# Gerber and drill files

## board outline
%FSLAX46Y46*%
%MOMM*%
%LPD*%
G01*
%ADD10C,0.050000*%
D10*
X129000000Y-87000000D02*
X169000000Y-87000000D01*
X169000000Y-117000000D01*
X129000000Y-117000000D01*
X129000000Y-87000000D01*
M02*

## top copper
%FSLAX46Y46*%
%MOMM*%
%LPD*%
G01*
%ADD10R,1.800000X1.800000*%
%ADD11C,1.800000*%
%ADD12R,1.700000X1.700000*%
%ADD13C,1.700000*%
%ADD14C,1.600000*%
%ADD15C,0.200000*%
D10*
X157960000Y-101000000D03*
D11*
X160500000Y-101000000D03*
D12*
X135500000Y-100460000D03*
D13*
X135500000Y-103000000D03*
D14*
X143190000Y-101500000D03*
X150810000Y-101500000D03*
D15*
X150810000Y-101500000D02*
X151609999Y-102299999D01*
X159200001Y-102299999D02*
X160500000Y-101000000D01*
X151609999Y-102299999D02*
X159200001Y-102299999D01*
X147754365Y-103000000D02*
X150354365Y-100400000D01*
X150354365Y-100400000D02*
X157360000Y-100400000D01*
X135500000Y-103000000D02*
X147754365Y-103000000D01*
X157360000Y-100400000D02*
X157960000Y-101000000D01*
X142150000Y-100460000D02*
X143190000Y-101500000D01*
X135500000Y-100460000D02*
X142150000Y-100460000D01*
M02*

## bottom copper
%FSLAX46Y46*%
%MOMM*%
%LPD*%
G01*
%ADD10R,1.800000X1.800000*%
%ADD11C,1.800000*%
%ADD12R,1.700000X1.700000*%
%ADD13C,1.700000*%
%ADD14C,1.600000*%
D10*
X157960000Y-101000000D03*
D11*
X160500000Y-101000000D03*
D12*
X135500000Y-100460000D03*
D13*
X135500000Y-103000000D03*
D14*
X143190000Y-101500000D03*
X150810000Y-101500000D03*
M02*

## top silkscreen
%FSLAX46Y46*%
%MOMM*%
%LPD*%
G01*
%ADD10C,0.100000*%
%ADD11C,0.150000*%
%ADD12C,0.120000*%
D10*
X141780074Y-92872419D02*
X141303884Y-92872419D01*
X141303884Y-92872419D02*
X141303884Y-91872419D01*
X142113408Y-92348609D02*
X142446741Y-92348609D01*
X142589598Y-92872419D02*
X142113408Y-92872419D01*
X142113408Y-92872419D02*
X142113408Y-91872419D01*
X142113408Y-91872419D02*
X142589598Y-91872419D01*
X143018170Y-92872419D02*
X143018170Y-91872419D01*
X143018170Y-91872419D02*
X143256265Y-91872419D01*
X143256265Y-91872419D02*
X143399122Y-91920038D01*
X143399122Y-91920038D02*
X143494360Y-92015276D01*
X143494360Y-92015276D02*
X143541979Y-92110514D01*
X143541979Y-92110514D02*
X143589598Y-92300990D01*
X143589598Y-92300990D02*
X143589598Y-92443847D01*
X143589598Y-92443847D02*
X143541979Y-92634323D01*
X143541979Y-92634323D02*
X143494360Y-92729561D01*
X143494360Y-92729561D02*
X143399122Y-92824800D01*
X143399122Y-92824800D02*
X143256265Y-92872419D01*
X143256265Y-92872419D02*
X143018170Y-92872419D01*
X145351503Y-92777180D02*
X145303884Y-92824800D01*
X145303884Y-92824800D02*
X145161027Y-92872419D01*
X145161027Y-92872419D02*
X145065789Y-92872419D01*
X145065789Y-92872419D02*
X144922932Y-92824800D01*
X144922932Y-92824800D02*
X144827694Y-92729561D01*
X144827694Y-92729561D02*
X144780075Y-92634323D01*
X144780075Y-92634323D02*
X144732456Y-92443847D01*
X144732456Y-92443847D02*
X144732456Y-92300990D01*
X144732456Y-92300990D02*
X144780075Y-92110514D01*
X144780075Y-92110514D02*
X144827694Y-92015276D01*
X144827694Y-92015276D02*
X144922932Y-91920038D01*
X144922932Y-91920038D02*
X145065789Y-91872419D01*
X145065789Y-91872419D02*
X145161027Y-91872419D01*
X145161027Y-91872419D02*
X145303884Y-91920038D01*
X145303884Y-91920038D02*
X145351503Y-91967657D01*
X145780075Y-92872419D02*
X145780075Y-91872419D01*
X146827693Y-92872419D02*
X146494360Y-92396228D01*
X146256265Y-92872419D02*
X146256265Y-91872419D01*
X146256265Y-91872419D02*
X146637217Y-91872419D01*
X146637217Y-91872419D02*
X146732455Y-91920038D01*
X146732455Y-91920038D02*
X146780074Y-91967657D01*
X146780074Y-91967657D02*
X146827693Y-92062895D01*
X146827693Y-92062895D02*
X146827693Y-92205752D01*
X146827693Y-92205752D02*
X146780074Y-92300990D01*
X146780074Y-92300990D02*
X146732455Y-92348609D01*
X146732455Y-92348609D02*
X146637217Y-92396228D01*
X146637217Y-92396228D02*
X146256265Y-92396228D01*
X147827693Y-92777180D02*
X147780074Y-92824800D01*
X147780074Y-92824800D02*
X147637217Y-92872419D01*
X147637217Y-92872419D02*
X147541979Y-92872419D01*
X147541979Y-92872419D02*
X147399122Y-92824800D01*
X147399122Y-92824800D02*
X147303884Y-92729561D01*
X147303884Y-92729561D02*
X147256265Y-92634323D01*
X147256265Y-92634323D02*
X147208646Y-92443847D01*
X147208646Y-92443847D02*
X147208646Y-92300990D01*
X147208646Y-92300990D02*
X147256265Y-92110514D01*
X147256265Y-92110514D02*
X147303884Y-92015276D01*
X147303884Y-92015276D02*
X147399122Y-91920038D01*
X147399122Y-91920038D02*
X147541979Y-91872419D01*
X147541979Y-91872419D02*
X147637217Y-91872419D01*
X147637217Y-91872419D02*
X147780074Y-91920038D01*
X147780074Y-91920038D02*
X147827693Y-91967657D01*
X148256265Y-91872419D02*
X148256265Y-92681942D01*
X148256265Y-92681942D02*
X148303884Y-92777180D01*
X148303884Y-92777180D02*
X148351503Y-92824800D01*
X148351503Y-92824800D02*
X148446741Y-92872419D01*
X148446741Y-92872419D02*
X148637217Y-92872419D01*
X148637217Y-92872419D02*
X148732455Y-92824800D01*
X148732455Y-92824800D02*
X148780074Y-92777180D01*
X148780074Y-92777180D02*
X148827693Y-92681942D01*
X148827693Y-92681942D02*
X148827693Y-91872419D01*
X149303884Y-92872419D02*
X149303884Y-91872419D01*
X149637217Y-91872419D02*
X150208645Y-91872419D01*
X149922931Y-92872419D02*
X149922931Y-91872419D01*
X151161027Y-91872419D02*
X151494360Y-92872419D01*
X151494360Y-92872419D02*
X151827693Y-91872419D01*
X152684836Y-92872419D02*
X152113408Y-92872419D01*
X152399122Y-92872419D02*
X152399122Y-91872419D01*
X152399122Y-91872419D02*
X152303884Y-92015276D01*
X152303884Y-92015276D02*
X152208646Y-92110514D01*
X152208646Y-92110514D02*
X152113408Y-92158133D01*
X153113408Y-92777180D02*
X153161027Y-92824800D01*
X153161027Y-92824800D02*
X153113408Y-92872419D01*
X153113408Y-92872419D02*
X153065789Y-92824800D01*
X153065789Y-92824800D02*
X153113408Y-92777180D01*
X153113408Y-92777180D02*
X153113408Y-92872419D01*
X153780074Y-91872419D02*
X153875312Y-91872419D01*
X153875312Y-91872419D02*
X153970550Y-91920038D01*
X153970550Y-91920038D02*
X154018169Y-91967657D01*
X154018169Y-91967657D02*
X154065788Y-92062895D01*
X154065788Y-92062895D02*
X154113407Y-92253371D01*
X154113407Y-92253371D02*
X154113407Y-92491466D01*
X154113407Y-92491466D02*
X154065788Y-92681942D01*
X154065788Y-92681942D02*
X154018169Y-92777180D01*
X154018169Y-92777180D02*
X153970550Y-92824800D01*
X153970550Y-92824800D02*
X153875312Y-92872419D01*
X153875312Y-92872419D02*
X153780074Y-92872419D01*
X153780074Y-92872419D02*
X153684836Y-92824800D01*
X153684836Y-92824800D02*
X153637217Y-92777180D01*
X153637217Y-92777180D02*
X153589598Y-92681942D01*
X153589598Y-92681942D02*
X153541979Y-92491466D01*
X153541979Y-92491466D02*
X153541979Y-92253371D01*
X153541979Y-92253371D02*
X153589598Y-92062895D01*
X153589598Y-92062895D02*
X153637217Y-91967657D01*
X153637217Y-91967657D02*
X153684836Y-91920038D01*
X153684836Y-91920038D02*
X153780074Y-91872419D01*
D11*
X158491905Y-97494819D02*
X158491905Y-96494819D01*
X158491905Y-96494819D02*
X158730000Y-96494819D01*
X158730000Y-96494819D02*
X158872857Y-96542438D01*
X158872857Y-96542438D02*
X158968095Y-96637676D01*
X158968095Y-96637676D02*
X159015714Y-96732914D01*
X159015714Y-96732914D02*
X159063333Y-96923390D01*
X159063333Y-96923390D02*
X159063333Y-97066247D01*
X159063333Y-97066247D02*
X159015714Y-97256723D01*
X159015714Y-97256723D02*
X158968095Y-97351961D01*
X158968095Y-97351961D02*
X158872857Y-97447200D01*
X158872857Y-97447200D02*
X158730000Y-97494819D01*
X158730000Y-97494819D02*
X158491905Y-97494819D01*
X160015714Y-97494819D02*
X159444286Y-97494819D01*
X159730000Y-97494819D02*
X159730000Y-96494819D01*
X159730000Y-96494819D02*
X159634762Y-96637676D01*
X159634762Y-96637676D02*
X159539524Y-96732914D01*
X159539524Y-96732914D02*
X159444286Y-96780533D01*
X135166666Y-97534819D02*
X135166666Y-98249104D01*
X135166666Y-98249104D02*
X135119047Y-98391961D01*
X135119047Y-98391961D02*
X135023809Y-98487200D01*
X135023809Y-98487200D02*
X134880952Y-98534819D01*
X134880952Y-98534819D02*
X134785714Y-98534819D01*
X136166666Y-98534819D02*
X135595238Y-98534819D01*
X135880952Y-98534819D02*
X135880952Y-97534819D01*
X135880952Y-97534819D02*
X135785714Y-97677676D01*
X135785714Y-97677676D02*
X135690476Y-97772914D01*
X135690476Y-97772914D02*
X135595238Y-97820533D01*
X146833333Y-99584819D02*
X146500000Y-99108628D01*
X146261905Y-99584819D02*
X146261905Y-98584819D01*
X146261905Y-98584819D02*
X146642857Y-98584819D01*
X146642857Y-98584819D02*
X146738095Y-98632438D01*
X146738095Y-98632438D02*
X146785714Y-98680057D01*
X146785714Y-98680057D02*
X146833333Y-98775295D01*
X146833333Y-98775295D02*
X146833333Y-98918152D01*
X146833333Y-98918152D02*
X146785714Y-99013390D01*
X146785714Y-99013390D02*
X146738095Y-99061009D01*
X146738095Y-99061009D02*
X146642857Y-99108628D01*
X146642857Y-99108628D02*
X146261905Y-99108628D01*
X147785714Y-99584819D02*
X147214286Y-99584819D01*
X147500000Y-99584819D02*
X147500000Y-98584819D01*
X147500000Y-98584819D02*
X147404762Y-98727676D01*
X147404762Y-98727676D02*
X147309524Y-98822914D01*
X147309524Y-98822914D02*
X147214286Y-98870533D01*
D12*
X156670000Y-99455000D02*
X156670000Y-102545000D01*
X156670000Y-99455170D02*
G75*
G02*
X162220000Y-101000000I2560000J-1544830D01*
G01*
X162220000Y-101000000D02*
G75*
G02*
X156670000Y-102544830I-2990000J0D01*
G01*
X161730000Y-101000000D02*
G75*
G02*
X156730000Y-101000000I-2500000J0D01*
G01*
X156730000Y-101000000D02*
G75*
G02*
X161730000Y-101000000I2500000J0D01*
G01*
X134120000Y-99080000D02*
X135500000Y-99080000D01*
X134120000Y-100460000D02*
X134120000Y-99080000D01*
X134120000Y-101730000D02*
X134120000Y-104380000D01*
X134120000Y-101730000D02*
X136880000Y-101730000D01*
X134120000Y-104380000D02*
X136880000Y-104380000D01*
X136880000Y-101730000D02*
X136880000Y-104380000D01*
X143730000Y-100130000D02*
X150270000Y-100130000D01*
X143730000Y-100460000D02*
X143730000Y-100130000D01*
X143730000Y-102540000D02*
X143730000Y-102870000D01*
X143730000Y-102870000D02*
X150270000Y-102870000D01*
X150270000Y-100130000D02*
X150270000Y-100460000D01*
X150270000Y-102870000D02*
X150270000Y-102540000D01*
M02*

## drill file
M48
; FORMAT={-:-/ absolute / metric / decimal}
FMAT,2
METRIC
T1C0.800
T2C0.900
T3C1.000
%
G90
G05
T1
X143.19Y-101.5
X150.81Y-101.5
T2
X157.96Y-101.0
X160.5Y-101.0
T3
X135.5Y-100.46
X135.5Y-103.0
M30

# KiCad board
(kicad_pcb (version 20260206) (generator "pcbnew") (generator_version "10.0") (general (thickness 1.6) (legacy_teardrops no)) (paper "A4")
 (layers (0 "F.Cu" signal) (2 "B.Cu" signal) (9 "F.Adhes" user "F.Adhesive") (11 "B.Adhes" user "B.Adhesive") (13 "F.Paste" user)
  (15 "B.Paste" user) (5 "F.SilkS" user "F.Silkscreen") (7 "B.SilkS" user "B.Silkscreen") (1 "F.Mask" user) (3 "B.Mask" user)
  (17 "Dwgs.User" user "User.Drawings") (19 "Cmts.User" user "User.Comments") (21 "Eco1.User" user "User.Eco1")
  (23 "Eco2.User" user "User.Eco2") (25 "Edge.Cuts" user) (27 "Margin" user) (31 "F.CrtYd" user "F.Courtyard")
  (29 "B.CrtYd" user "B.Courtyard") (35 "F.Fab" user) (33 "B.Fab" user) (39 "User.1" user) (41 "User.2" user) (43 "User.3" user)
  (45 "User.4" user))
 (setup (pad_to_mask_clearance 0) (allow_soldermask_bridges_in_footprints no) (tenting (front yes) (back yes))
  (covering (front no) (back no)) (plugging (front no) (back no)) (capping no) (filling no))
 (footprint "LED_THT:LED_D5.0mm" (layer "F.Cu") (at 157.96 101)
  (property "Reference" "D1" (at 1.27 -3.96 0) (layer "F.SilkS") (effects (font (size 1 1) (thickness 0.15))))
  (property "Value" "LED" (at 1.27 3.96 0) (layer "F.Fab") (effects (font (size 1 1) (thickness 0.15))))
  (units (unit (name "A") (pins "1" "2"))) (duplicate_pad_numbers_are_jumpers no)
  (fp_line (start -1.29 -1.545) (end -1.29 1.545) (stroke (width 0.12) (type solid)) (layer "F.SilkS"))
  (fp_arc (start -1.29 -1.54483) (mid 2.071779 -2.880495) (end 4.26 0) (stroke (width 0.12) (type solid)) (layer "F.SilkS"))
  (fp_arc (start 4.26 0) (mid 2.071779 2.880495) (end -1.29 1.54483) (stroke (width 0.12) (type solid)) (layer "F.SilkS"))
  (fp_circle (center 1.27 0) (end 3.77 0) (stroke (width 0.12) (type solid)) (fill no) (layer "F.SilkS"))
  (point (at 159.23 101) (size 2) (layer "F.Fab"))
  (pad "1" thru_hole rect (at 0 0) (size 1.8 1.8) (drill 0.9) (layers "*.Cu" "*.Mask") (remove_unused_layers no) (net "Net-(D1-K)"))
  (pad "2" thru_hole circle (at 2.54 0) (size 1.8 1.8) (drill 0.9) (layers "*.Cu" "*.Mask") (remove_unused_layers no) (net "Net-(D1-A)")))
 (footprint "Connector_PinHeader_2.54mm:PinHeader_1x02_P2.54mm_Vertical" (layer "F.Cu") (at 135.5 100.46)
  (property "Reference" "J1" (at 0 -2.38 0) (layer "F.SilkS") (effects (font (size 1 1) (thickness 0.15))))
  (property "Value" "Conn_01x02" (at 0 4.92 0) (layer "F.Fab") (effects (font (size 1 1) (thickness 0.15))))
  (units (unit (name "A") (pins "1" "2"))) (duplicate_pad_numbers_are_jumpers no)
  (fp_line (start -1.38 -1.38) (end 0 -1.38) (stroke (width 0.12) (type solid)) (layer "F.SilkS"))
  (fp_line (start -1.38 0) (end -1.38 -1.38) (stroke (width 0.12) (type solid)) (layer "F.SilkS"))
  (fp_line (start -1.38 1.27) (end -1.38 3.92) (stroke (width 0.12) (type solid)) (layer "F.SilkS"))
  (fp_line (start -1.38 1.27) (end 1.38 1.27) (stroke (width 0.12) (type solid)) (layer "F.SilkS"))
  (fp_line (start -1.38 3.92) (end 1.38 3.92) (stroke (width 0.12) (type solid)) (layer "F.SilkS"))
  (fp_line (start 1.38 1.27) (end 1.38 3.92) (stroke (width 0.12) (type solid)) (layer "F.SilkS"))
  (pad "1" thru_hole rect (at 0 0) (size 1.7 1.7) (drill 1) (layers "*.Cu" "*.Mask") (remove_unused_layers no) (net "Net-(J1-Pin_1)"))
  (pad "2" thru_hole circle (at 0 2.54) (size 1.7 1.7) (drill 1) (layers "*.Cu" "*.Mask") (remove_unused_layers no) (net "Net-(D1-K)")))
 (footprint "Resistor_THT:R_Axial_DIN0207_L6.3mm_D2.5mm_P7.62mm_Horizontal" (layer "F.Cu") (at 143.19 101.5)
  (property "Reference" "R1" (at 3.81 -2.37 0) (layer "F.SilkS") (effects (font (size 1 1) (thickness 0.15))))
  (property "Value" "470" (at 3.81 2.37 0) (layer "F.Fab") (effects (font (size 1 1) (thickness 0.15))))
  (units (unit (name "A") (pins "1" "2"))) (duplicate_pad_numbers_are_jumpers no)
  (fp_line (start 0.54 -1.37) (end 7.08 -1.37) (stroke (width 0.12) (type solid)) (layer "F.SilkS"))
  (fp_line (start 0.54 -1.04) (end 0.54 -1.37) (stroke (width 0.12) (type solid)) (layer "F.SilkS"))
  (fp_line (start 0.54 1.04) (end 0.54 1.37) (stroke (width 0.12) (type solid)) (layer "F.SilkS"))
  (fp_line (start 0.54 1.37) (end 7.08 1.37) (stroke (width 0.12) (type solid)) (layer "F.SilkS"))
  (fp_line (start 7.08 -1.37) (end 7.08 -1.04) (stroke (width 0.12) (type solid)) (layer "F.SilkS"))
  (fp_line (start 7.08 1.37) (end 7.08 1.04) (stroke (width 0.12) (type solid)) (layer "F.SilkS"))
  (pad "1" thru_hole circle (at 0 0) (size 1.6 1.6) (drill 0.8) (layers "*.Cu" "*.Mask") (remove_unused_layers no) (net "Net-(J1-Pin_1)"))
  (pad "2" thru_hole circle (at 7.62 0) (size 1.6 1.6) (drill 0.8) (layers "*.Cu" "*.Mask") (remove_unused_layers no) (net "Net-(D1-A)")))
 (gr_rect (start 129 87) (end 169 117) (stroke (width 0.05) (type solid)) (fill no) (layer "Edge.Cuts"))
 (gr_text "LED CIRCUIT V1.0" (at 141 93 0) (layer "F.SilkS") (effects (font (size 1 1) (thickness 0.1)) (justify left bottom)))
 (segment (start 150.81 101.5) (end 151.609999 102.299999) (width 0.2) (layer "F.Cu") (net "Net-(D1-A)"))
 (segment (start 159.200001 102.299999) (end 160.5 101) (width 0.2) (layer "F.Cu") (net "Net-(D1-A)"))
 (segment (start 151.609999 102.299999) (end 159.200001 102.299999) (width 0.2) (layer "F.Cu") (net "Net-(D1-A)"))
 (segment (start 147.754365 103) (end 150.354365 100.4) (width 0.2) (layer "F.Cu") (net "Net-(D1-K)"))
 (segment (start 150.354365 100.4) (end 157.36 100.4) (width 0.2) (layer "F.Cu") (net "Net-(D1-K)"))
 (segment (start 135.5 103) (end 147.754365 103) (width 0.2) (layer "F.Cu") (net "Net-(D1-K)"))
 (segment (start 157.36 100.4) (end 157.96 101) (width 0.2) (layer "F.Cu") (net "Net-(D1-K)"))
 (segment (start 142.15 100.46) (end 143.19 101.5) (width 0.2) (layer "F.Cu") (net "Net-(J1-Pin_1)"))
 (segment (start 135.5 100.46) (end 142.15 100.46) (width 0.2) (layer "F.Cu") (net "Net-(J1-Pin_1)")))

